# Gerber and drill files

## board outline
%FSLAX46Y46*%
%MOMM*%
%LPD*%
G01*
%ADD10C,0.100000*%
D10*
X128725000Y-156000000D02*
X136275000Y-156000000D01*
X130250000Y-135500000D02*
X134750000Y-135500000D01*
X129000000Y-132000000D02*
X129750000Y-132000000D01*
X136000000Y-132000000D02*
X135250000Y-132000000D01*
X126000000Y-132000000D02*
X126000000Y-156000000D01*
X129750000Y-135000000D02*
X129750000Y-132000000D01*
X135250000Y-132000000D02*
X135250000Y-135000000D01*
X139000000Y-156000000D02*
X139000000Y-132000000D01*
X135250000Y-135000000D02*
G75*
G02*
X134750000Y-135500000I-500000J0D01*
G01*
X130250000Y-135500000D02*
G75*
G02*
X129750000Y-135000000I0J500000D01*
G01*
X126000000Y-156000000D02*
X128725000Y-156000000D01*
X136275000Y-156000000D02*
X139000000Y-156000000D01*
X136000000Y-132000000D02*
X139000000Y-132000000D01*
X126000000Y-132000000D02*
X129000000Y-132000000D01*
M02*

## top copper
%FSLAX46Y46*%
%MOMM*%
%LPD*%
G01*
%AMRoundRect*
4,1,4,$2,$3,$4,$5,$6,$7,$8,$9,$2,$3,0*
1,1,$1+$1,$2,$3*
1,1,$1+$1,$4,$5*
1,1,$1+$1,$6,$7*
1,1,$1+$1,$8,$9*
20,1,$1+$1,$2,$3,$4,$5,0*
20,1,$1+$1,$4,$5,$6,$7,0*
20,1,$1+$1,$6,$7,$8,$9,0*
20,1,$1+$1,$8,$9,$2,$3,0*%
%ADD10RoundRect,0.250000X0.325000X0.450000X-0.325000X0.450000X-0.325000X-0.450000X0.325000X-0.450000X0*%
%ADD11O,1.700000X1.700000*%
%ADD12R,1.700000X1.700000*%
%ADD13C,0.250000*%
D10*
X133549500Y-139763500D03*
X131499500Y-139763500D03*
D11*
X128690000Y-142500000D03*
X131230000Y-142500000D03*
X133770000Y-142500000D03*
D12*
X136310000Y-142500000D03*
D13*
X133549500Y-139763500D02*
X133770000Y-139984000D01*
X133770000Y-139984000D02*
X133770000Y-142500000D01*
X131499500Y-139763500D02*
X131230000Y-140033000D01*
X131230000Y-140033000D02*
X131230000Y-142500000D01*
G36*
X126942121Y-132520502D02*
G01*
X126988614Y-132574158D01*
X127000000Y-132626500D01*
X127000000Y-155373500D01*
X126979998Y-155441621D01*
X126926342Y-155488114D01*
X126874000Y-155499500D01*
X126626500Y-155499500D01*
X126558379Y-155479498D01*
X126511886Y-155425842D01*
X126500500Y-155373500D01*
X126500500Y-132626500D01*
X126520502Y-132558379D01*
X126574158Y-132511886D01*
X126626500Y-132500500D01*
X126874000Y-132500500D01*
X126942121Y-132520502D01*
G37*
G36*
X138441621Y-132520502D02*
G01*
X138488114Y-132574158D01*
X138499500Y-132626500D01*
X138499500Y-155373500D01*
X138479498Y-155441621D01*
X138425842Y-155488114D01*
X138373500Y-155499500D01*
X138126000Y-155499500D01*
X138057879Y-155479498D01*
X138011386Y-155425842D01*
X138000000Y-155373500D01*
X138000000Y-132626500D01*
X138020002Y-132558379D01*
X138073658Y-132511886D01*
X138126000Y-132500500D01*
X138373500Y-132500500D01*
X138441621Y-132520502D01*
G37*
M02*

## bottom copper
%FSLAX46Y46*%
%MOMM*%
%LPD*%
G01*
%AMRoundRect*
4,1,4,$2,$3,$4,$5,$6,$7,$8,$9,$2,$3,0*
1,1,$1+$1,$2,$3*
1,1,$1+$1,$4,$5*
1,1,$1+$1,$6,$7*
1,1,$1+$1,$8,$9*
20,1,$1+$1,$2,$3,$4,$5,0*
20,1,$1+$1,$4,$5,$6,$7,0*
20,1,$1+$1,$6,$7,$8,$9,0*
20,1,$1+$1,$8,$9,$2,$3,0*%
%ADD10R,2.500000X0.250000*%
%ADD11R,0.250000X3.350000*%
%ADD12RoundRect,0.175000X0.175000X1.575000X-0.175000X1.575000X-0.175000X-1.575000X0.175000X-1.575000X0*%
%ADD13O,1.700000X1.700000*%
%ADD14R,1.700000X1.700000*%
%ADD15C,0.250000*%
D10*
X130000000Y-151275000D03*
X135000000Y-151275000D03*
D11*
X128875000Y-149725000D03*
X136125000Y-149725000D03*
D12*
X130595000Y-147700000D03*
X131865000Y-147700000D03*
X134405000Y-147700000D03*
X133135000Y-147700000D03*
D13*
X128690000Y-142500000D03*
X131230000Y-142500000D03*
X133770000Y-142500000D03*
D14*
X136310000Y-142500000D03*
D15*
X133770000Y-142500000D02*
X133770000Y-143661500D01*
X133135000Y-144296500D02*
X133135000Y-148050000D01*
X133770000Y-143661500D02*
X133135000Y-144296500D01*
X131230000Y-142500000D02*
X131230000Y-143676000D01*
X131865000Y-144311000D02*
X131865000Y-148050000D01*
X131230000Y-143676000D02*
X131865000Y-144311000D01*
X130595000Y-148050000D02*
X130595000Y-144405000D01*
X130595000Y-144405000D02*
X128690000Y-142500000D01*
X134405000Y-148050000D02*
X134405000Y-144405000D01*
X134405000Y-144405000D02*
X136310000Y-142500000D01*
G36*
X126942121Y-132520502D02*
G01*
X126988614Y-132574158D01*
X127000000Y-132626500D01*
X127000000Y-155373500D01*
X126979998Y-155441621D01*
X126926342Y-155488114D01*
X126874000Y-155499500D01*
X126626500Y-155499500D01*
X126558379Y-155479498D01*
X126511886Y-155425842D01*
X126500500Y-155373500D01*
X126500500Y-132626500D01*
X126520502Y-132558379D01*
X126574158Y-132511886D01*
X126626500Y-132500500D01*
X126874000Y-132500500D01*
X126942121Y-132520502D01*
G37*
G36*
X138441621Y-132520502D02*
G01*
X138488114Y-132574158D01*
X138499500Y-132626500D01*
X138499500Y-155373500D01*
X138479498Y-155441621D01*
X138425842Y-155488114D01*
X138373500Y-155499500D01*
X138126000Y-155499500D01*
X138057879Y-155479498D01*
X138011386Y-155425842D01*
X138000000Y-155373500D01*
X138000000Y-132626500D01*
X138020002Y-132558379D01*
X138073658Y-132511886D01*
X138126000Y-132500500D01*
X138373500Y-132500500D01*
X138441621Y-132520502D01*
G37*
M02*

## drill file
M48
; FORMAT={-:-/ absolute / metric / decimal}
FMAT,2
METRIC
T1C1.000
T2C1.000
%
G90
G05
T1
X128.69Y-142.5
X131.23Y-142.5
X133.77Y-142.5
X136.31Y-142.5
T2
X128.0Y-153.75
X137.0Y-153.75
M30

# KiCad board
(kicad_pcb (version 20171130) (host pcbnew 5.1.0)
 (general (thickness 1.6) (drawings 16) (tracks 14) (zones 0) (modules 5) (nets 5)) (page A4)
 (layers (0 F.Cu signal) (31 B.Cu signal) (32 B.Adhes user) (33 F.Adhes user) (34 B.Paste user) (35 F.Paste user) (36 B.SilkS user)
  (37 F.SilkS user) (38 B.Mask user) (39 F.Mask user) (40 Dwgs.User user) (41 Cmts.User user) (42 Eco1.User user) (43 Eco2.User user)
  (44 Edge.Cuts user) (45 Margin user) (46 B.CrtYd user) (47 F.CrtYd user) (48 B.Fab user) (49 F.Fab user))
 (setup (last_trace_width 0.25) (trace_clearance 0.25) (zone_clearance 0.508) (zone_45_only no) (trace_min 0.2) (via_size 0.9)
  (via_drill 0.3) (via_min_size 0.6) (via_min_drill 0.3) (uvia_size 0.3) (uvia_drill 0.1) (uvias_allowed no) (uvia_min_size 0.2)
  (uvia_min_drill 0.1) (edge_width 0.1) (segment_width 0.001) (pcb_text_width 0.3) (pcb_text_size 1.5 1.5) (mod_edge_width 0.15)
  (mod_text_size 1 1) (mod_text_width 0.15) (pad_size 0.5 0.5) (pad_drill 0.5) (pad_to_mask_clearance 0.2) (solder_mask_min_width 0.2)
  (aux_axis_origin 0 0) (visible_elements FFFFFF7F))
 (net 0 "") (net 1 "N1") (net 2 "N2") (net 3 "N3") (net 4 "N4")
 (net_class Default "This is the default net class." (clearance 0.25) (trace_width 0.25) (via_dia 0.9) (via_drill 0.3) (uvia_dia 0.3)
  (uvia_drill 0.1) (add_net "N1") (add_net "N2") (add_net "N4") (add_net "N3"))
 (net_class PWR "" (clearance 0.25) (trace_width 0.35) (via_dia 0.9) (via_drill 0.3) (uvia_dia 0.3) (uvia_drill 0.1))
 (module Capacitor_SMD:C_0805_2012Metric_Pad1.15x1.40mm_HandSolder (layer F.Cu) (at 132.5245 139.7635 180)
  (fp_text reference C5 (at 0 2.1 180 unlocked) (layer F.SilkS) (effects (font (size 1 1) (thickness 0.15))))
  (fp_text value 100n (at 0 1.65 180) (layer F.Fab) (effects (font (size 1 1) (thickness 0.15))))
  (pad 1 smd roundrect (at -1.025 0 180) (size 1.15 1.4) (layers F.Cu F.Paste F.Mask) (roundrect_rratio 0.217391) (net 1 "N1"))
  (pad 2 smd roundrect (at 1.025 0 180) (size 1.15 1.4) (layers F.Cu F.Paste F.Mask) (roundrect_rratio 0.217391) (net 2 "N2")))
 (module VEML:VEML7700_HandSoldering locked (layer B.Cu) (at 132.5 150 180)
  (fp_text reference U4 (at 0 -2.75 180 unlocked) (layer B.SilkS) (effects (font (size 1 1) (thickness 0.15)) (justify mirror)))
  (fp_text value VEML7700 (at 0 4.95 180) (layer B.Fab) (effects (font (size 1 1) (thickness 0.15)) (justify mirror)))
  (pad ~ smd rect (at 2.5 -1.275 180) (size 2.5 0.25) (layers B.Cu B.Paste B.Mask))
  (pad ~ smd rect (at -2.5 -1.275 180) (size 2.5 0.25) (layers B.Cu B.Paste B.Mask))
  (pad ~ smd rect (at 3.625 0.45 180) (size 0.25 3.35) (drill (offset 0 -0.175)) (layers B.Cu B.Paste B.Mask))
  (pad ~ smd rect (at -3.625 0.45 180) (size 0.25 3.35) (drill (offset 0 -0.175)) (layers B.Cu B.Paste B.Mask))
  (pad 1 smd roundrect (at 1.905 1.95 180) (size 0.7 3.5) (drill (offset 0 0.35)) (layers B.Cu B.Paste B.Mask) (roundrect_rratio 0.25)
   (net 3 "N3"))
  (pad 2 smd roundrect (at 0.635 1.95 180) (size 0.7 3.5) (drill (offset 0 0.35)) (layers B.Cu B.Paste B.Mask) (roundrect_rratio 0.25)
   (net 2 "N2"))
  (pad 4 smd roundrect (at -1.905 1.95 180) (size 0.7 3.5) (drill (offset 0 0.35)) (layers B.Cu B.Paste B.Mask) (roundrect_rratio 0.25)
   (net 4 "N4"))
  (pad 3 smd roundrect (at -0.635 1.95 180) (size 0.7 3.5) (drill (offset 0 0.35)) (layers B.Cu B.Paste B.Mask) (roundrect_rratio 0.25)
   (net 1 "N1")))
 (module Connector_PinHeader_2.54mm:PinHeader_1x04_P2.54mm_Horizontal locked (layer B.Cu) (at 136.31 142.5 90)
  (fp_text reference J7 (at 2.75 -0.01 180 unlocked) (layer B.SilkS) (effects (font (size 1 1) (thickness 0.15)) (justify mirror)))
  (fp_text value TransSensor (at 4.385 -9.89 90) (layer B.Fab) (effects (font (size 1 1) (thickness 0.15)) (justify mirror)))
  (pad 4 thru_hole oval (at 0 -7.62 90) (size 1.7 1.7) (drill 1) (layers *.Cu *.Mask) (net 3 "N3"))
  (pad 3 thru_hole oval (at 0 -5.08 90) (size 1.7 1.7) (drill 1) (layers *.Cu *.Mask) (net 2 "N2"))
  (pad 2 thru_hole oval (at 0 -2.54 90) (size 1.7 1.7) (drill 1) (layers *.Cu *.Mask) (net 1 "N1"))
  (pad 1 thru_hole rect (at 0 0 90) (size 1.7 1.7) (drill 1) (layers *.Cu *.Mask) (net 4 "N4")))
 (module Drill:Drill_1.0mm (layer F.Cu) (at 128 153.75)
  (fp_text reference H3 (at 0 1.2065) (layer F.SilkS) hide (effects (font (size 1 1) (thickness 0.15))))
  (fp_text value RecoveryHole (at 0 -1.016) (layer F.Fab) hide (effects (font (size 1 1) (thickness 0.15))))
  (pad "" np_thru_hole circle (at 0 0) (size 1 1) (drill 1) (layers *.Cu *.Mask) (solder_mask_margin 0.0001) (clearance 0.25)))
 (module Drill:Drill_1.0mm (layer F.Cu) (at 137 153.75)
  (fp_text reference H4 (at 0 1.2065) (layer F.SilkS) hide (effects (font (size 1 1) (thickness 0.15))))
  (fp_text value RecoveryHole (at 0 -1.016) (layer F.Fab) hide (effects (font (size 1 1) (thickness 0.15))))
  (pad "" np_thru_hole circle (at 0 0) (size 1 1) (drill 1) (layers *.Cu *.Mask) (solder_mask_margin 0.0001) (clearance 0.25)))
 (gr_line (start 128.725 156) (end 136.275 156) (layer Edge.Cuts) (width 0.1))
 (gr_line (start 130.25 135.5) (end 134.75 135.5) (layer Edge.Cuts) (width 0.1))
 (gr_line (start 129 132) (end 129.75 132) (layer Edge.Cuts) (width 0.1))
 (gr_line (start 136 132) (end 135.25 132) (layer Edge.Cuts) (width 0.1))
 (gr_line (start 126 132) (end 126 156) (layer Edge.Cuts) (width 0.1))
 (gr_line (start 129.75 135) (end 129.75 132) (layer Edge.Cuts) (width 0.1))
 (gr_line (start 135.25 132) (end 135.25 135) (layer Edge.Cuts) (width 0.1))
 (gr_line (start 139 156) (end 139 132) (layer Edge.Cuts) (width 0.1))
 (gr_arc (start 134.75 135) (end 134.75 135.5) (angle -90) (layer Edge.Cuts) (width 0.1))
 (gr_arc (start 130.25 135) (end 129.75 135) (angle -90) (layer Edge.Cuts) (width 0.1))
 (gr_line (start 126 156) (end 128.725 156) (angle 90) (layer Edge.Cuts) (width 0.1))
 (gr_line (start 136.275 156) (end 139 156) (angle 90) (layer Edge.Cuts) (width 0.1))
 (gr_line (start 136 132) (end 139 132) (angle 90) (layer Edge.Cuts) (width 0.1))
 (gr_line (start 126 132) (end 129 132) (angle 90) (layer Edge.Cuts) (width 0.1))
 (segment (start 133.5495 139.7635) (end 133.77 139.984) (width 0.25) (layer F.Cu) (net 1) (status C00000))
 (segment (start 133.77 139.984) (end 133.77 142.5) (width 0.25) (layer F.Cu) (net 1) (status C00000))
 (segment (start 133.77 142.5) (end 133.77 143.6615) (width 0.25) (layer B.Cu) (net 1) (status 400000))
 (segment (start 133.135 144.2965) (end 133.135 148.05) (width 0.25) (layer B.Cu) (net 1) (status 800000))
 (segment (start 133.77 143.6615) (end 133.135 144.2965) (width 0.25) (layer B.Cu) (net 1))
 (segment (start 131.4995 139.7635) (end 131.23 140.033) (width 0.25) (layer F.Cu) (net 2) (status C00000))
 (segment (start 131.23 140.033) (end 131.23 142.5) (width 0.25) (layer F.Cu) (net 2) (status C00000))
 (segment (start 131.23 142.5) (end 131.23 143.676) (width 0.25) (layer B.Cu) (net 2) (status 400000))
 (segment (start 131.865 144.311) (end 131.865 148.05) (width 0.25) (layer B.Cu) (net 2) (status 800000))
 (segment (start 131.23 143.676) (end 131.865 144.311) (width 0.25) (layer B.Cu) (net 2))
 (segment (start 130.595 148.05) (end 130.595 144.405) (width 0.25) (layer B.Cu) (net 3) (status 400000))
 (segment (start 130.595 144.405) (end 128.69 142.5) (width 0.25) (layer B.Cu) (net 3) (status 800000))
 (segment (start 134.405 148.05) (end 134.405 144.405) (width 0.25) (layer B.Cu) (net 4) (status 400000))
 (segment (start 134.405 144.405) (end 136.31 142.5) (width 0.25) (layer B.Cu) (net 4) (status 800000))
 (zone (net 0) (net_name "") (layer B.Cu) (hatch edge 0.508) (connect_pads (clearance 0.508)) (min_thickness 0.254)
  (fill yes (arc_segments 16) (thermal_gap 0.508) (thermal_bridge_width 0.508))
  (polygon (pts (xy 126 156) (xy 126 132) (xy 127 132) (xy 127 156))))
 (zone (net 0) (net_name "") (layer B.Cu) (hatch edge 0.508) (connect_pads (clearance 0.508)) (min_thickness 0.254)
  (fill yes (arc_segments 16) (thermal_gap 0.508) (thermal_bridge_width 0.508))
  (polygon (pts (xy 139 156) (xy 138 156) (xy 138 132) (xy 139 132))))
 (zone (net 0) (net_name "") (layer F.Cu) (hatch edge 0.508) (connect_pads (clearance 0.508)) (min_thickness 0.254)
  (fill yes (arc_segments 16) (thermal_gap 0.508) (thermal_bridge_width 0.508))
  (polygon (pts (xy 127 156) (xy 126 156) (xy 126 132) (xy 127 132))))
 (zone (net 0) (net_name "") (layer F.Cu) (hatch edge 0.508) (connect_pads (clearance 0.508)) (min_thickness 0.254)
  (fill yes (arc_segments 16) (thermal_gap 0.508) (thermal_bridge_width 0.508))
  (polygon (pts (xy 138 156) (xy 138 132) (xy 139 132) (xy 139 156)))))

